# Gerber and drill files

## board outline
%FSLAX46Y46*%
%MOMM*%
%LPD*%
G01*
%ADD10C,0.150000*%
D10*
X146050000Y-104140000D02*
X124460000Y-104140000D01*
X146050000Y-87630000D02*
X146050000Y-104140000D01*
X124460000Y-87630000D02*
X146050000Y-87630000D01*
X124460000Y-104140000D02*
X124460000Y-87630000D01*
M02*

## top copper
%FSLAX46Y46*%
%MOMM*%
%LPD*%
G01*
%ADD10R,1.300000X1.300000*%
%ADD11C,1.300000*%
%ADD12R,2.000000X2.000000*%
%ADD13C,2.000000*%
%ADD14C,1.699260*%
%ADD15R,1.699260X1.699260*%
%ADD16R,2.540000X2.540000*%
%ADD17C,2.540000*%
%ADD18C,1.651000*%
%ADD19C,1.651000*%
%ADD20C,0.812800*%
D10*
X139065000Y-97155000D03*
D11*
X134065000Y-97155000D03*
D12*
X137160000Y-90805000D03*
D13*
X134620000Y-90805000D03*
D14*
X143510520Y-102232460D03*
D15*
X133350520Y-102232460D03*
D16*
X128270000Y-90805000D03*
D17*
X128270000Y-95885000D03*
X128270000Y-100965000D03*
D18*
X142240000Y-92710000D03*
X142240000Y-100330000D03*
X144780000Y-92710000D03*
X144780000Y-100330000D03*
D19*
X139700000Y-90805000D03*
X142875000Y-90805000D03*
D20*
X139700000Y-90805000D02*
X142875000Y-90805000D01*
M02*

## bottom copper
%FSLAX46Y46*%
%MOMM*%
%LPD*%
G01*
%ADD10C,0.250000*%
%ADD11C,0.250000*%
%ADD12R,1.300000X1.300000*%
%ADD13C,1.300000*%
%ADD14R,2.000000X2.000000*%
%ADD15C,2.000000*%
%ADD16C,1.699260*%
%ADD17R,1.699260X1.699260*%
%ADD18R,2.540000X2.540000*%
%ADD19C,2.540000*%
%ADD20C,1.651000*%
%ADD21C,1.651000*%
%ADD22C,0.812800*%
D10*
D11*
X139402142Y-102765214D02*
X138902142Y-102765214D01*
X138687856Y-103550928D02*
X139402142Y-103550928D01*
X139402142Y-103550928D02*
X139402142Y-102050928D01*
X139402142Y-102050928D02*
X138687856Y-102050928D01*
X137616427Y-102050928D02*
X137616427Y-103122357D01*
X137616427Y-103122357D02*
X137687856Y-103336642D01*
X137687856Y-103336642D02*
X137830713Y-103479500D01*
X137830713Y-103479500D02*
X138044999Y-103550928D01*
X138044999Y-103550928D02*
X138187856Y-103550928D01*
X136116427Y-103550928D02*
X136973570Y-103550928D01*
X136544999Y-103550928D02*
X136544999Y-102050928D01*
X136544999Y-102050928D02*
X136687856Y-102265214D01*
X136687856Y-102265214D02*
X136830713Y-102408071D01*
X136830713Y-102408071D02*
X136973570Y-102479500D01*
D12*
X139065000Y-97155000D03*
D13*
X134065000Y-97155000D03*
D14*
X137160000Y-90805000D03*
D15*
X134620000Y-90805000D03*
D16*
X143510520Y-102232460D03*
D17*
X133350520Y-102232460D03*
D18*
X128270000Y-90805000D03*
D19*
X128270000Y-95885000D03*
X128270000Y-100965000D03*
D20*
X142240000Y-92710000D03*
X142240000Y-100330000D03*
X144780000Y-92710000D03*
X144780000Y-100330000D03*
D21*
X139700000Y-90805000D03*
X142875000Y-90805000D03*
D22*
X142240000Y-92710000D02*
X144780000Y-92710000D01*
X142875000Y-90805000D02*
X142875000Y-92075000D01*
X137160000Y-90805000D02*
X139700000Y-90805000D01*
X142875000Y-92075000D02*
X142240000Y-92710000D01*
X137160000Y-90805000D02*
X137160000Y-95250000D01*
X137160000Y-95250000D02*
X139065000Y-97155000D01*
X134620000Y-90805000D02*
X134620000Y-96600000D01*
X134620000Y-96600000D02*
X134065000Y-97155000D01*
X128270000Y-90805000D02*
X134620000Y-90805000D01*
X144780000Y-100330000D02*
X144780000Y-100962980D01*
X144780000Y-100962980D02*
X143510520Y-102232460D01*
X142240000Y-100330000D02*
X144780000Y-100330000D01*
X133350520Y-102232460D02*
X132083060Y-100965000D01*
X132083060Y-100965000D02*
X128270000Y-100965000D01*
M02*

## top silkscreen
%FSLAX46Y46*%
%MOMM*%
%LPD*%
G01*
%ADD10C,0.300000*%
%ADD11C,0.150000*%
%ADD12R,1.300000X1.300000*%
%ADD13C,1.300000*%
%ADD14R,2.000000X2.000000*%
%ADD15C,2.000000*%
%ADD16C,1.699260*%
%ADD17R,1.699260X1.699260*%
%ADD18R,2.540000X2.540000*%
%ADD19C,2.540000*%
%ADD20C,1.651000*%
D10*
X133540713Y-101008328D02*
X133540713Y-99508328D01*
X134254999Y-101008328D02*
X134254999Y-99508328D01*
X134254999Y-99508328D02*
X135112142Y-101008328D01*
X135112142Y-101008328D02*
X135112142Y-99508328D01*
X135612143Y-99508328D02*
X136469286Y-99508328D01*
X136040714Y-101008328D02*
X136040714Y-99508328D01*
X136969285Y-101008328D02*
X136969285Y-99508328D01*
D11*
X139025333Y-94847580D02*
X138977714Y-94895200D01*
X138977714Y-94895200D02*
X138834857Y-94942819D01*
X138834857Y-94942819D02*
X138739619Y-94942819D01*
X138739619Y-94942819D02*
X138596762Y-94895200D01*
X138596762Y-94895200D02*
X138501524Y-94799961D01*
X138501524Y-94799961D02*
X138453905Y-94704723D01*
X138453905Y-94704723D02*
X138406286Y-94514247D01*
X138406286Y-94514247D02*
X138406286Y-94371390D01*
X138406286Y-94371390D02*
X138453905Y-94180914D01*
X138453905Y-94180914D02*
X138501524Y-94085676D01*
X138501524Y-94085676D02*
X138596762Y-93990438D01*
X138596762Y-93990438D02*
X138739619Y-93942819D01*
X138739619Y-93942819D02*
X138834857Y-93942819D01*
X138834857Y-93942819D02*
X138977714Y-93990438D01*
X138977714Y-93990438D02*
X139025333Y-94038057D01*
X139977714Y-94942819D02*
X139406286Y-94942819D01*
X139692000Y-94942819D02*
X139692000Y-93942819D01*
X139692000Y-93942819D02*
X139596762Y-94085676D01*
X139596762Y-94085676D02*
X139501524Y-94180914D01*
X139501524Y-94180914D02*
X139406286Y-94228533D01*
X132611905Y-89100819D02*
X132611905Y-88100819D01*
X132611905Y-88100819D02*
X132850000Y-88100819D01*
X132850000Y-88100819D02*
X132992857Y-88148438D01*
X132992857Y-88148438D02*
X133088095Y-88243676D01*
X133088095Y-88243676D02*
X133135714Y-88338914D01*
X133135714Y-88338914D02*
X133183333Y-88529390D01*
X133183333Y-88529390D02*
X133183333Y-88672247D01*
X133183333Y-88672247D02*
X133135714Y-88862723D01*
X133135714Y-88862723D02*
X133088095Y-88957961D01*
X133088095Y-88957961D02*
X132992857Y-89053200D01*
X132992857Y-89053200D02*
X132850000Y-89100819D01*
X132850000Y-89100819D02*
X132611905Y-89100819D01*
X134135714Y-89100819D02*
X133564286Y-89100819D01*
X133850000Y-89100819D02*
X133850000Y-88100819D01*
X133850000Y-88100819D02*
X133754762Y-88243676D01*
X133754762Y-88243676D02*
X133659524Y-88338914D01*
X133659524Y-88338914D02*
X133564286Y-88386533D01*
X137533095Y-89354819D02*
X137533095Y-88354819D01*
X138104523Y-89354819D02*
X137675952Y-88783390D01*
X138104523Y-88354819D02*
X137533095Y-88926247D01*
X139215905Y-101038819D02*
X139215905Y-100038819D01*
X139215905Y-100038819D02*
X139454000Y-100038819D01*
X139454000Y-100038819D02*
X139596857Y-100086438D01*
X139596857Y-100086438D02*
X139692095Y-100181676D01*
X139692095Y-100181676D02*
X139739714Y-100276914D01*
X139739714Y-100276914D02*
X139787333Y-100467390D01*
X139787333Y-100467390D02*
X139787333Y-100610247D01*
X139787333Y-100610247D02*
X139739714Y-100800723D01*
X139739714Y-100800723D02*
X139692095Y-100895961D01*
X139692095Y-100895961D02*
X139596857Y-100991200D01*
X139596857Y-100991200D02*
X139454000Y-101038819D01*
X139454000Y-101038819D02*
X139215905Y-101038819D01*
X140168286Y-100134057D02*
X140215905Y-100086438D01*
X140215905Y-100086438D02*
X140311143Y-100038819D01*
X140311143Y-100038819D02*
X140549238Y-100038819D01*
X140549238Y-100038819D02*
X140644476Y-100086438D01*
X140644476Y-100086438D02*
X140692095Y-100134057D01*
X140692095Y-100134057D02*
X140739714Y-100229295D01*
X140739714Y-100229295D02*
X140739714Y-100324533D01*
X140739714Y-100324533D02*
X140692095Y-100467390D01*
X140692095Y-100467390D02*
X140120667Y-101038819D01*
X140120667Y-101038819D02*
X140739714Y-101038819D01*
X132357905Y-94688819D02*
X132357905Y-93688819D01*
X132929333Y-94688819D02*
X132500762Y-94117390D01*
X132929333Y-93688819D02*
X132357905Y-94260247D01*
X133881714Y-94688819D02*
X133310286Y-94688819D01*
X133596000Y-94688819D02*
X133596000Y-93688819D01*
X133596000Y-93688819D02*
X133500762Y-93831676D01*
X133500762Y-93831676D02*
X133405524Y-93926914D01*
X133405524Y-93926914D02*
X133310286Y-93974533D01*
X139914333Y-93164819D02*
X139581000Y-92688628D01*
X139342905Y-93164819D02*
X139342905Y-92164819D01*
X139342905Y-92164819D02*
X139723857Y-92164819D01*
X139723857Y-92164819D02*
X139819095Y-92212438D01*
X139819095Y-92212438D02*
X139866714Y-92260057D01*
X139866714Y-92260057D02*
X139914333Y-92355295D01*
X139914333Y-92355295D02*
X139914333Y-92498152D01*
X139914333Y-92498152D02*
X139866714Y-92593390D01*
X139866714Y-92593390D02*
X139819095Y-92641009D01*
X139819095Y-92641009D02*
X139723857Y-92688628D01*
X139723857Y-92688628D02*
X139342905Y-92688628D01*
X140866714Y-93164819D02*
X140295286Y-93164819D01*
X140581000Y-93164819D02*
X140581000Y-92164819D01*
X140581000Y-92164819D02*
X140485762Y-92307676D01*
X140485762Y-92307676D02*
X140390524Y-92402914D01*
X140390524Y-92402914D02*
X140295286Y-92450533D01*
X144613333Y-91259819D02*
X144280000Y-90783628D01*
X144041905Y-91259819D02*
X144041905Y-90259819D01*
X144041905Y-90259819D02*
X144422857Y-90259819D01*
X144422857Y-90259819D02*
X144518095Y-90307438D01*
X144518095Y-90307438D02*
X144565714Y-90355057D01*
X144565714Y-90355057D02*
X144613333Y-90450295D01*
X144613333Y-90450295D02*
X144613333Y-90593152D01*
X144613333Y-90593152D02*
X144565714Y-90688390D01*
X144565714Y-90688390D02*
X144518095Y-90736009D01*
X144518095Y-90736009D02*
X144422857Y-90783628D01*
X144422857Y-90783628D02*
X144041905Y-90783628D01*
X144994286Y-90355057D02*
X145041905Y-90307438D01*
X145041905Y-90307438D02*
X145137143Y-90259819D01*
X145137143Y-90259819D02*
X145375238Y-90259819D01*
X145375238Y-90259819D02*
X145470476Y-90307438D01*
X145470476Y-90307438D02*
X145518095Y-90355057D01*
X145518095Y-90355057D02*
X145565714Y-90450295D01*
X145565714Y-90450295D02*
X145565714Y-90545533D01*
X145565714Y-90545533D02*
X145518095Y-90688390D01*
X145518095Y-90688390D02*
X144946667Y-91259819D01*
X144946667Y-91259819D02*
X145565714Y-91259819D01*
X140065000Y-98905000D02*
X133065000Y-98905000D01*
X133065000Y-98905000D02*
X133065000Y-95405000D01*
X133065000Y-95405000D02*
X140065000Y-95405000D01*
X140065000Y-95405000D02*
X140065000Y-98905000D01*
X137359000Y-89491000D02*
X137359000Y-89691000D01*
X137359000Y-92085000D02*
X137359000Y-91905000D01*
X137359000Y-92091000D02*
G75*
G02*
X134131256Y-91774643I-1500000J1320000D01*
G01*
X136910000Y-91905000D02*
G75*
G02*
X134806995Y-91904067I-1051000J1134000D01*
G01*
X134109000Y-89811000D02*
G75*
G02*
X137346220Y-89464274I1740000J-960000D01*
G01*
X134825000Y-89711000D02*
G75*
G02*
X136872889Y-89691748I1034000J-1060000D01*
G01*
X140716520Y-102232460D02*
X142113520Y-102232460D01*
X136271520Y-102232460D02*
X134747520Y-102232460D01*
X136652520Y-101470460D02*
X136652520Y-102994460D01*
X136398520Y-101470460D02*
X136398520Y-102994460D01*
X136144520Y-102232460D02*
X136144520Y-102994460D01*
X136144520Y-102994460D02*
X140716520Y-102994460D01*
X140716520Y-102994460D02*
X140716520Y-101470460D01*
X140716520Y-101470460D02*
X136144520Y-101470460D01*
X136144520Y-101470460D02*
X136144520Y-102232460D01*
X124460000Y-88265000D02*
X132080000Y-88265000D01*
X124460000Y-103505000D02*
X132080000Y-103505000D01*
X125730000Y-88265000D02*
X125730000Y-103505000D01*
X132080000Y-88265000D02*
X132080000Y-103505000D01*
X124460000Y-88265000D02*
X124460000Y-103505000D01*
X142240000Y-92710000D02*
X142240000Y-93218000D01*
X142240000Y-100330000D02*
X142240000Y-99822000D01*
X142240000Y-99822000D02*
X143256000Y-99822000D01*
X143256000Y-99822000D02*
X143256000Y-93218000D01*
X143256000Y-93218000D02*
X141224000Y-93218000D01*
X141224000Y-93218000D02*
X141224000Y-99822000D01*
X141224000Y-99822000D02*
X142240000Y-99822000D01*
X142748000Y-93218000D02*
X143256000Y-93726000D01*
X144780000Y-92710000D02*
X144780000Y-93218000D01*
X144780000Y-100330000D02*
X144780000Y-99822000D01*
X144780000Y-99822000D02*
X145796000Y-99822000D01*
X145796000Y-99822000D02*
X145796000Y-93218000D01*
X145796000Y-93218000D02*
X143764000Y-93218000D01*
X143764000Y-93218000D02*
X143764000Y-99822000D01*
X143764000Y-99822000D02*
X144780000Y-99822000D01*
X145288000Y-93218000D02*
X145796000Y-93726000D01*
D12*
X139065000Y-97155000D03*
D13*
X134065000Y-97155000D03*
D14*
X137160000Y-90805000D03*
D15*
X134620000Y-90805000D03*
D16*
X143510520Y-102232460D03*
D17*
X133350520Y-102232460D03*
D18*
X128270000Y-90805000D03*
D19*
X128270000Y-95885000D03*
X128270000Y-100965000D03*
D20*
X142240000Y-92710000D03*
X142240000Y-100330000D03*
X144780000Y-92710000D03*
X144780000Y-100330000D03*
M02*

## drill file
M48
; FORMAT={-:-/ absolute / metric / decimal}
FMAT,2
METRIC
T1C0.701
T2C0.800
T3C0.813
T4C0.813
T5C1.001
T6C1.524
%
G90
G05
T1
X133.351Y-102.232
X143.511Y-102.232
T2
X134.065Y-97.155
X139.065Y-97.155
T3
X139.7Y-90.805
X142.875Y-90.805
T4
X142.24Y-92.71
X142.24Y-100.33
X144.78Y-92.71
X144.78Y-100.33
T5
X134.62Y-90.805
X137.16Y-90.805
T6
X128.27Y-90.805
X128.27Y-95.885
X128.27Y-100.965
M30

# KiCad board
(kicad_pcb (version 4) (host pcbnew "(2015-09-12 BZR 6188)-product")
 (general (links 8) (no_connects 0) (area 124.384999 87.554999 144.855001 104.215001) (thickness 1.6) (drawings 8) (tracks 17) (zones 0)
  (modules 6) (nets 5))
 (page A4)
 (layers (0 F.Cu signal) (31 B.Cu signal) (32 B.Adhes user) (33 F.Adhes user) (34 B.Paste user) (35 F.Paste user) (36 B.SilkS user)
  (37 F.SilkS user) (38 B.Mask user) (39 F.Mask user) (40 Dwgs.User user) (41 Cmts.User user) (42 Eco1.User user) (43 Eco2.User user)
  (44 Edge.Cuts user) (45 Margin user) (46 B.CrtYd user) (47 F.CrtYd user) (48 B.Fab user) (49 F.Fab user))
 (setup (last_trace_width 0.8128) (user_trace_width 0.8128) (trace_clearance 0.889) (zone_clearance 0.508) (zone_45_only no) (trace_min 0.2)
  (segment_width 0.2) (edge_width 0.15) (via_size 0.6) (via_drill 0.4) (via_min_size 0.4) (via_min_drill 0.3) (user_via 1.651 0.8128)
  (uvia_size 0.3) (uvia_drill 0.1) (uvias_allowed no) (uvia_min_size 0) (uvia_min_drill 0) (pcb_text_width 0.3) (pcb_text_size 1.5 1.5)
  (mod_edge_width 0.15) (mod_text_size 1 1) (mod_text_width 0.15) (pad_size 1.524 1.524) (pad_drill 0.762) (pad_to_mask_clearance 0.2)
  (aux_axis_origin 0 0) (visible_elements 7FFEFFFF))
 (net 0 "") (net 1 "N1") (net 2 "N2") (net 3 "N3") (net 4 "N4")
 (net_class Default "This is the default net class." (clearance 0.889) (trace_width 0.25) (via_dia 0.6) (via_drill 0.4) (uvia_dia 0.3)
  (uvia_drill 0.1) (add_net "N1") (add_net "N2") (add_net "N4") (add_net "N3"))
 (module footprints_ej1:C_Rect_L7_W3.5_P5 (layer F.Cu) (at 139.065 97.155 180)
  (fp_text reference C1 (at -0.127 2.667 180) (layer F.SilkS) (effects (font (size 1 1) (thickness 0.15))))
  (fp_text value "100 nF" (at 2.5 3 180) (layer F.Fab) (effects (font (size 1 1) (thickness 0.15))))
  (fp_line (start -1 -1.75) (end 6 -1.75) (layer F.SilkS) (width 0.15))
  (fp_line (start 6 -1.75) (end 6 1.75) (layer F.SilkS) (width 0.15))
  (fp_line (start 6 1.75) (end -1 1.75) (layer F.SilkS) (width 0.15))
  (fp_line (start -1 1.75) (end -1 -1.75) (layer F.SilkS) (width 0.15))
  (pad 1 thru_hole rect (at 0 0 180) (size 1.3 1.3) (drill 0.8) (layers *.Cu *.Mask F.SilkS) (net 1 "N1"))
  (pad 2 thru_hole circle (at 5 0 180) (size 1.3 1.3) (drill 0.8) (layers *.Cu *.Mask F.SilkS) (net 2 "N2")))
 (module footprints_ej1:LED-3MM (layer F.Cu) (at 137.16 90.805 180)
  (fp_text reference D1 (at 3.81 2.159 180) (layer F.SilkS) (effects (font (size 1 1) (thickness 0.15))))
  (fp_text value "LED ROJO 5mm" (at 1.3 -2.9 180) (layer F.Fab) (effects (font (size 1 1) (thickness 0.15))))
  (fp_line (start -0.199 1.314) (end -0.199 1.114) (layer F.SilkS) (width 0.15))
  (fp_line (start -0.199 -1.28) (end -0.199 -1.1) (layer F.SilkS) (width 0.15))
  (fp_arc (start 1.301 0.034) (end -0.199 -1.286) (angle 108.5) (layer F.SilkS) (width 0.15))
  (fp_arc (start 1.301 0.034) (end 0.25 -1.1) (angle 85.7) (layer F.SilkS) (width 0.15))
  (fp_arc (start 1.311 0.034) (end 3.051 0.994) (angle 110) (layer F.SilkS) (width 0.15))
  (fp_arc (start 1.301 0.034) (end 2.335 1.094) (angle 87.5) (layer F.SilkS) (width 0.15))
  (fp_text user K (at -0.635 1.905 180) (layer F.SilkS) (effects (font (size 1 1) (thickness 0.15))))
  (pad 1 thru_hole rect (at 0 0 270) (size 2 2) (drill 1.00076) (layers *.Cu *.Mask F.SilkS) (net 1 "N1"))
  (pad 2 thru_hole circle (at 2.54 0 180) (size 2 2) (drill 1.00076) (layers *.Cu *.Mask F.SilkS) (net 2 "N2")))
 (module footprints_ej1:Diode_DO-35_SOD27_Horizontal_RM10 (layer F.Cu) (at 133.35 102.235)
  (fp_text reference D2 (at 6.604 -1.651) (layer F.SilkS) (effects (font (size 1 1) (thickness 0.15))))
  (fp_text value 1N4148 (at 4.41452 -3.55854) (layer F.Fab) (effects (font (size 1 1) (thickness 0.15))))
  (fp_line (start 7.36652 -0.00254) (end 8.76352 -0.00254) (layer F.SilkS) (width 0.15))
  (fp_line (start 2.92152 -0.00254) (end 1.39752 -0.00254) (layer F.SilkS) (width 0.15))
  (fp_line (start 3.30252 -0.76454) (end 3.30252 0.75946) (layer F.SilkS) (width 0.15))
  (fp_line (start 3.04852 -0.76454) (end 3.04852 0.75946) (layer F.SilkS) (width 0.15))
  (fp_line (start 2.79452 -0.00254) (end 2.79452 0.75946) (layer F.SilkS) (width 0.15))
  (fp_line (start 2.79452 0.75946) (end 7.36652 0.75946) (layer F.SilkS) (width 0.15))
  (fp_line (start 7.36652 0.75946) (end 7.36652 -0.76454) (layer F.SilkS) (width 0.15))
  (fp_line (start 7.36652 -0.76454) (end 2.79452 -0.76454) (layer F.SilkS) (width 0.15))
  (fp_line (start 2.79452 -0.76454) (end 2.79452 -0.00254) (layer F.SilkS) (width 0.15))
  (pad 2 thru_hole circle (at 10.16052 -0.00254 180) (size 1.69926 1.69926) (drill 0.70104) (layers *.Cu *.Mask F.SilkS) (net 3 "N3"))
  (pad 1 thru_hole rect (at 0.00052 -0.00254 180) (size 1.69926 1.69926) (drill 0.70104) (layers *.Cu *.Mask F.SilkS) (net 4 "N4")))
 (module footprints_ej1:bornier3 (layer F.Cu) (at 128.27 95.885 270)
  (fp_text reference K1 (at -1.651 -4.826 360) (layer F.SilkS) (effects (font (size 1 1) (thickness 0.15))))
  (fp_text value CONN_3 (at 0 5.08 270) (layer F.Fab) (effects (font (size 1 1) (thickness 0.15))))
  (fp_line (start -7.62 3.81) (end -7.62 -3.81) (layer F.SilkS) (width 0.15))
  (fp_line (start 7.62 3.81) (end 7.62 -3.81) (layer F.SilkS) (width 0.15))
  (fp_line (start -7.62 2.54) (end 7.62 2.54) (layer F.SilkS) (width 0.15))
  (fp_line (start -7.62 -3.81) (end 7.62 -3.81) (layer F.SilkS) (width 0.15))
  (fp_line (start -7.62 3.81) (end 7.62 3.81) (layer F.SilkS) (width 0.15))
  (pad 1 thru_hole rect (at -5.08 0 270) (size 2.54 2.54) (drill 1.524) (layers *.Cu *.Mask F.SilkS) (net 2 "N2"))
  (pad 2 thru_hole circle (at 0 0 270) (size 2.54 2.54) (drill 1.524) (layers *.Cu *.Mask F.SilkS))
  (pad 3 thru_hole circle (at 5.08 0 270) (size 2.54 2.54) (drill 1.524) (layers *.Cu *.Mask F.SilkS) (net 4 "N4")))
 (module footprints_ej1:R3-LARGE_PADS (layer F.Cu) (at 142.24 96.52 270)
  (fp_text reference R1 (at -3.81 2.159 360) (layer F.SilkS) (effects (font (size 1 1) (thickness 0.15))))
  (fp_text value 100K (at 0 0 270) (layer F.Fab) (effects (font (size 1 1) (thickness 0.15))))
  (fp_line (start -3.81 0) (end -3.302 0) (layer F.SilkS) (width 0.15))
  (fp_line (start 3.81 0) (end 3.302 0) (layer F.SilkS) (width 0.15))
  (fp_line (start 3.302 0) (end 3.302 -1.016) (layer F.SilkS) (width 0.15))
  (fp_line (start 3.302 -1.016) (end -3.302 -1.016) (layer F.SilkS) (width 0.15))
  (fp_line (start -3.302 -1.016) (end -3.302 1.016) (layer F.SilkS) (width 0.15))
  (fp_line (start -3.302 1.016) (end 3.302 1.016) (layer F.SilkS) (width 0.15))
  (fp_line (start 3.302 1.016) (end 3.302 0) (layer F.SilkS) (width 0.15))
  (fp_line (start -3.302 -0.508) (end -2.794 -1.016) (layer F.SilkS) (width 0.15))
  (pad 1 thru_hole circle (at -3.81 0 270) (size 1.651 1.651) (drill 0.8128) (layers *.Cu *.Mask F.SilkS) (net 1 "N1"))
  (pad 2 thru_hole circle (at 3.81 0 270) (size 1.651 1.651) (drill 0.8128) (layers *.Cu *.Mask F.SilkS) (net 3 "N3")))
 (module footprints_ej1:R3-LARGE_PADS (layer F.Cu) (at 144.78 96.52 270)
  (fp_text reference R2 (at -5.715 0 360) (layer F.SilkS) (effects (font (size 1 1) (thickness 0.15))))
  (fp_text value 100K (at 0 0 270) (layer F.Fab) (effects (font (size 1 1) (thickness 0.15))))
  (fp_line (start -3.81 0) (end -3.302 0) (layer F.SilkS) (width 0.15))
  (fp_line (start 3.81 0) (end 3.302 0) (layer F.SilkS) (width 0.15))
  (fp_line (start 3.302 0) (end 3.302 -1.016) (layer F.SilkS) (width 0.15))
  (fp_line (start 3.302 -1.016) (end -3.302 -1.016) (layer F.SilkS) (width 0.15))
  (fp_line (start -3.302 -1.016) (end -3.302 1.016) (layer F.SilkS) (width 0.15))
  (fp_line (start -3.302 1.016) (end 3.302 1.016) (layer F.SilkS) (width 0.15))
  (fp_line (start 3.302 1.016) (end 3.302 0) (layer F.SilkS) (width 0.15))
  (fp_line (start -3.302 -0.508) (end -2.794 -1.016) (layer F.SilkS) (width 0.15))
  (pad 1 thru_hole circle (at -3.81 0 270) (size 1.651 1.651) (drill 0.8128) (layers *.Cu *.Mask F.SilkS) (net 1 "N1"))
  (pad 2 thru_hole circle (at 3.81 0 270) (size 1.651 1.651) (drill 0.8128) (layers *.Cu *.Mask F.SilkS) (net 3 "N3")))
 (gr_line (start 146.05 104.14) (end 124.46 104.14) (angle 90) (layer Edge.Cuts) (width 0.15))
 (gr_line (start 146.05 87.63) (end 146.05 104.14) (angle 90) (layer Edge.Cuts) (width 0.15))
 (gr_line (start 124.46 87.63) (end 146.05 87.63) (angle 90) (layer Edge.Cuts) (width 0.15))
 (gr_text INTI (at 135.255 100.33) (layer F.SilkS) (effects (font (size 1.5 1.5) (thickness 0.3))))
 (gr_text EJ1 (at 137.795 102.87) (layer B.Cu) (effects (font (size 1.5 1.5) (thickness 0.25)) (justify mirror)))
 (gr_line (start 124.46 104.14) (end 124.46 87.63) (angle 90) (layer Edge.Cuts) (width 0.15))
 (segment (start 142.24 92.71) (end 144.78 92.71) (width 0.8128) (layer B.Cu) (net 1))
 (segment (start 142.875 90.805) (end 142.875 92.075) (width 0.8128) (layer B.Cu) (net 1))
 (via (at 139.7 90.805) (size 1.651) (drill 0.8128) (layers F.Cu B.Cu) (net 1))
 (segment (start 139.7 90.805) (end 142.875 90.805) (width 0.8128) (layer F.Cu) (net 1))
 (via (at 142.875 90.805) (size 1.651) (drill 0.8128) (layers F.Cu B.Cu) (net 1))
 (segment (start 137.16 90.805) (end 139.7 90.805) (width 0.8128) (layer B.Cu) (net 1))
 (segment (start 142.875 92.075) (end 142.24 92.71) (width 0.8128) (layer B.Cu) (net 1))
 (segment (start 137.16 90.805) (end 137.16 95.25) (width 0.8128) (layer B.Cu) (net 1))
 (segment (start 137.16 95.25) (end 139.065 97.155) (width 0.8128) (layer B.Cu) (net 1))
 (segment (start 134.62 90.805) (end 134.62 96.6) (width 0.8128) (layer B.Cu) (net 2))
 (segment (start 134.62 96.6) (end 134.065 97.155) (width 0.8128) (layer B.Cu) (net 2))
 (segment (start 128.27 90.805) (end 134.62 90.805) (width 0.8128) (layer B.Cu) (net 2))
 (segment (start 144.78 100.33) (end 144.78 100.96298) (width 0.8128) (layer B.Cu) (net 3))
 (segment (start 144.78 100.96298) (end 143.51052 102.23246) (width 0.8128) (layer B.Cu) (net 3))
 (segment (start 142.24 100.33) (end 144.78 100.33) (width 0.8128) (layer B.Cu) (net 3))
 (segment (start 133.35052 102.23246) (end 132.08306 100.965) (width 0.8128) (layer B.Cu) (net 4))
 (segment (start 132.08306 100.965) (end 128.27 100.965) (width 0.8128) (layer B.Cu) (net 4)))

